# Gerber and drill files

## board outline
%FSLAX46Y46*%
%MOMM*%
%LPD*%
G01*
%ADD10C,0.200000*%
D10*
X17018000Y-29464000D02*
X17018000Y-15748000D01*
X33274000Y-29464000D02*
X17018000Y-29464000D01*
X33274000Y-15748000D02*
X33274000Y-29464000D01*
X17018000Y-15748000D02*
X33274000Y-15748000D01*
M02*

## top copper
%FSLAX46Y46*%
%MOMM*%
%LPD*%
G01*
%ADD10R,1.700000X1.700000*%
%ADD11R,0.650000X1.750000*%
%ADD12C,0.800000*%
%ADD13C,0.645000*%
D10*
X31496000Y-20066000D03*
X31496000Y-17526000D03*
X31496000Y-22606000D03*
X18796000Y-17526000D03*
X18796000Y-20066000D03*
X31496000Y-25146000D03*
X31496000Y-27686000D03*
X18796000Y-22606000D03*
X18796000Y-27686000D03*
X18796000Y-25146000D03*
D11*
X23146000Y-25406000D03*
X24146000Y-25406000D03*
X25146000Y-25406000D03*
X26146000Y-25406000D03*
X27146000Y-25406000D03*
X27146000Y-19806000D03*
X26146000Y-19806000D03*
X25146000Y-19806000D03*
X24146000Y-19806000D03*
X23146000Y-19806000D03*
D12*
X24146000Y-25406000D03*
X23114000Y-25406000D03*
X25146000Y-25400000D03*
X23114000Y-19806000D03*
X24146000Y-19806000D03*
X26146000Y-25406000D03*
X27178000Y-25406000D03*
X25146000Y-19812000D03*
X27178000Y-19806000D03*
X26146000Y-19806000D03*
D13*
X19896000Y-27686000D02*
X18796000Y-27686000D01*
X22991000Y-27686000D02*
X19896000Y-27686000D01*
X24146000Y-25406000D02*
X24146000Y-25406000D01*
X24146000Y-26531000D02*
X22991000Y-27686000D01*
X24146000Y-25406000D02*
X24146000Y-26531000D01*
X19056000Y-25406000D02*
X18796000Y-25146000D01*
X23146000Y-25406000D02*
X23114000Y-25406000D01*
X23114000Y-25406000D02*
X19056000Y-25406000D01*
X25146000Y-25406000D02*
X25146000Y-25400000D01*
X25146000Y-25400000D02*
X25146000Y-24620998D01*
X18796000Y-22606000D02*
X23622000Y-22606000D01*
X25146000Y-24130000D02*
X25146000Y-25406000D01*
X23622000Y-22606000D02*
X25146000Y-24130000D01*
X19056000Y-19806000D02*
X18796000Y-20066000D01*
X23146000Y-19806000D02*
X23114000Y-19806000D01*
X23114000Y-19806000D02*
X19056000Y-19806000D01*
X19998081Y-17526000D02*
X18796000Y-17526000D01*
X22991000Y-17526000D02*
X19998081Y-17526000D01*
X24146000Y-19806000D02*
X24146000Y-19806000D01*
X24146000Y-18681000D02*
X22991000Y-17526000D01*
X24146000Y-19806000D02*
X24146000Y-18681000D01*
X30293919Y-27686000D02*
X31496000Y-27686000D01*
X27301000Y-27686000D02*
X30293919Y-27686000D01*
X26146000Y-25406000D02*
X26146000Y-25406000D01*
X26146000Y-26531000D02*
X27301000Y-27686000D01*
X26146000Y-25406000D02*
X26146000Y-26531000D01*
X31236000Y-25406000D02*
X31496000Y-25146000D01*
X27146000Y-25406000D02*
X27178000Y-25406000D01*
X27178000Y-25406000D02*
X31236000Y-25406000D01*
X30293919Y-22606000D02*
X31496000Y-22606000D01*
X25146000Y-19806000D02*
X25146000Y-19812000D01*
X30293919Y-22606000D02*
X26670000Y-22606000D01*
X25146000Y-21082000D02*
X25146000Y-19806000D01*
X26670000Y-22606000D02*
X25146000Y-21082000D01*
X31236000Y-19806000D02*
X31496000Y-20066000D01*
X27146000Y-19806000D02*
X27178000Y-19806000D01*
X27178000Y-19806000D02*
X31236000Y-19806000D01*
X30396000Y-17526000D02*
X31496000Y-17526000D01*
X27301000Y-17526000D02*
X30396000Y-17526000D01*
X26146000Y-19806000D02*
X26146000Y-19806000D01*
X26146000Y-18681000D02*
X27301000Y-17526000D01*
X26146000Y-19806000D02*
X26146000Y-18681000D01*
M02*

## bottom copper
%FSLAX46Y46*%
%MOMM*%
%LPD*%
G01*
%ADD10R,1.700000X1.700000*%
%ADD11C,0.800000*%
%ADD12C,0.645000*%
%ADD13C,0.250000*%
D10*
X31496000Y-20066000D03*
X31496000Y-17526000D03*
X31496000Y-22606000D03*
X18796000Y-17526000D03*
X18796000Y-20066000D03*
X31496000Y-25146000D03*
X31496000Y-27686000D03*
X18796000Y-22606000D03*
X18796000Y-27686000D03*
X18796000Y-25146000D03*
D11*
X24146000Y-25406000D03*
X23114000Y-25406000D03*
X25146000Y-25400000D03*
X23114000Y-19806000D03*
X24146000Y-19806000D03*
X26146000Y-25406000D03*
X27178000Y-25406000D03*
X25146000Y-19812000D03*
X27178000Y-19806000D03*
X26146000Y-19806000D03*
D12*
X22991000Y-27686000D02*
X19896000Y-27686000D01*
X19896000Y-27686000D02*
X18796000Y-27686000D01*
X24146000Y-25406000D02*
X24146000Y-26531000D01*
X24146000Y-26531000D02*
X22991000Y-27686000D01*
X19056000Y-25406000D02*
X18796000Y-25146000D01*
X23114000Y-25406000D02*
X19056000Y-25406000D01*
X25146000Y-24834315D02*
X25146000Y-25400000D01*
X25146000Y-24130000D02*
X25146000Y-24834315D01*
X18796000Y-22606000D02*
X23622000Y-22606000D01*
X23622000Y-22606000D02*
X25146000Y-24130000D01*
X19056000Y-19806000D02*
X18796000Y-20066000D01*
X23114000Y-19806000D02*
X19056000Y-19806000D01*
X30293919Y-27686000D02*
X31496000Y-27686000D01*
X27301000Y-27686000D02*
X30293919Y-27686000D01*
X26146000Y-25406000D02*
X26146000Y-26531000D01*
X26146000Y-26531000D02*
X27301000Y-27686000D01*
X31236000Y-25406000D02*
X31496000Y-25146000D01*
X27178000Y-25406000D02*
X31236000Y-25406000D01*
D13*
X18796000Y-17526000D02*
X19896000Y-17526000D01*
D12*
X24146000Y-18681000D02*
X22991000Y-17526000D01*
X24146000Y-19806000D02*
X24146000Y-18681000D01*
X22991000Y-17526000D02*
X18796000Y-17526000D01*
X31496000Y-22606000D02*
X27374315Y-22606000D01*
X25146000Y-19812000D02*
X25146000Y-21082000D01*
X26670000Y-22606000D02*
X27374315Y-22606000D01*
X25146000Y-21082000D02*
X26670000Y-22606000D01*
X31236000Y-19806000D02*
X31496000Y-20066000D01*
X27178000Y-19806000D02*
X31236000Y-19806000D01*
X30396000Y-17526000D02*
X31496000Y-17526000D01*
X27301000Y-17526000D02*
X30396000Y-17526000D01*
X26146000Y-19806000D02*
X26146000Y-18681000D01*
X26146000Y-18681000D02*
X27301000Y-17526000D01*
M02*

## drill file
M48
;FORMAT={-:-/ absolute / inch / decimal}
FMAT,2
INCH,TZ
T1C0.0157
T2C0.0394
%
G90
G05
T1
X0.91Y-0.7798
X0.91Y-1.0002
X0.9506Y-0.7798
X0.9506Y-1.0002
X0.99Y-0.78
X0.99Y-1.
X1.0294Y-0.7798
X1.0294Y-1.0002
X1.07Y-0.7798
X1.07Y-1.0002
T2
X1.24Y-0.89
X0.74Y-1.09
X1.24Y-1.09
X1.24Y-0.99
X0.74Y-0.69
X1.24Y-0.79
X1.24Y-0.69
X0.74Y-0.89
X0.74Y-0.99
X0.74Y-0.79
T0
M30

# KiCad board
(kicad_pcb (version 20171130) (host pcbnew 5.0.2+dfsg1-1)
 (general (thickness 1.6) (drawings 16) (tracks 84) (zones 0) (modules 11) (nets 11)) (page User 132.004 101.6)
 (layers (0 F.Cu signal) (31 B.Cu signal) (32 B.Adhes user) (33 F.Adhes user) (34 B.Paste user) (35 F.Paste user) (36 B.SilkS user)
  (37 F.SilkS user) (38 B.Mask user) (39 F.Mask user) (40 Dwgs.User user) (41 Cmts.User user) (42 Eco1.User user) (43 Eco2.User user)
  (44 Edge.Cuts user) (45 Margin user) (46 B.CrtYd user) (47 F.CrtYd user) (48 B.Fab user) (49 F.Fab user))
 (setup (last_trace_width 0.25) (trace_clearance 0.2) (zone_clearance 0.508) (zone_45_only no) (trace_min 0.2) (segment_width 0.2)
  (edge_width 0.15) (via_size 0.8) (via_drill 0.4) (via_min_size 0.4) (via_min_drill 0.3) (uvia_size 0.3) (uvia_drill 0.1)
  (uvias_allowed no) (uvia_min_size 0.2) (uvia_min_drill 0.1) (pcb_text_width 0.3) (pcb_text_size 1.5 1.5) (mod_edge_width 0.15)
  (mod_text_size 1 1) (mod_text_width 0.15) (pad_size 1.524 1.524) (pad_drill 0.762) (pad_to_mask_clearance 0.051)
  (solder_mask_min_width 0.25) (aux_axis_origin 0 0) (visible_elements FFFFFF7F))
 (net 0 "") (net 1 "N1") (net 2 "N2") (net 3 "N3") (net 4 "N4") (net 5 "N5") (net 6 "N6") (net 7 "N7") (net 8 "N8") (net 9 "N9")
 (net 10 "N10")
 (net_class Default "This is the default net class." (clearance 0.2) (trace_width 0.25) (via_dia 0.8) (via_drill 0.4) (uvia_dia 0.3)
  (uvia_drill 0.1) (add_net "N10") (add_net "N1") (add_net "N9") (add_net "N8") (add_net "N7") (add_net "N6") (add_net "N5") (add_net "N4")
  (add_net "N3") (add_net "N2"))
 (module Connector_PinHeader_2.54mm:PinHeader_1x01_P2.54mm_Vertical (layer F.Cu) (at 31.496 20.066)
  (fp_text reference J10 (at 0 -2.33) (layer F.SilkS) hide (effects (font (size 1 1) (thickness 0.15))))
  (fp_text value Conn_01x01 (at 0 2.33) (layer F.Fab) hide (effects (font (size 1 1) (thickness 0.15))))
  (pad 1 thru_hole rect (at 0 0) (size 1.7 1.7) (drill 1) (layers *.Cu *.Mask) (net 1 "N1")))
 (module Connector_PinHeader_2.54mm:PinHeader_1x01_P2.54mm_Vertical (layer F.Cu) (at 31.496 17.526)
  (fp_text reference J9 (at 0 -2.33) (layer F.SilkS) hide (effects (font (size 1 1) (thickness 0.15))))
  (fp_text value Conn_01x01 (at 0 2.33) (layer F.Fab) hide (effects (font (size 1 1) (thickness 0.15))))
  (pad 1 thru_hole rect (at 0 0) (size 1.7 1.7) (drill 1) (layers *.Cu *.Mask) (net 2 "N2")))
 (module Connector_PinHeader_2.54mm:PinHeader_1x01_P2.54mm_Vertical (layer F.Cu) (at 31.496 22.606)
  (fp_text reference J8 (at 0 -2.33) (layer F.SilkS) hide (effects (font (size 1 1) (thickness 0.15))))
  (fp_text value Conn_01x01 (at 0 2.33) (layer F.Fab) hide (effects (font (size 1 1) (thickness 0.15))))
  (pad 1 thru_hole rect (at 0 0) (size 1.7 1.7) (drill 1) (layers *.Cu *.Mask) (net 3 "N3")))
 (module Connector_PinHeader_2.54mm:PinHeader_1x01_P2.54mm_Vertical (layer F.Cu) (at 18.796 17.526)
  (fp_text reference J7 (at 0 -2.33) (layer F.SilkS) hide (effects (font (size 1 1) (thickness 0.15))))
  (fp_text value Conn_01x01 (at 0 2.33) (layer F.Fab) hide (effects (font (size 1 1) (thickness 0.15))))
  (pad 1 thru_hole rect (at 0 0) (size 1.7 1.7) (drill 1) (layers *.Cu *.Mask) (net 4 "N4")))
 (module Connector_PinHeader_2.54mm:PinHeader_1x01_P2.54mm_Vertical (layer F.Cu) (at 18.796 20.066)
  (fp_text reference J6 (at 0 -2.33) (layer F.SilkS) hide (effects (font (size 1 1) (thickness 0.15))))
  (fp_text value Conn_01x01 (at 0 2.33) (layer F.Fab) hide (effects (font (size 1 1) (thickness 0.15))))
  (pad 1 thru_hole rect (at 0 0) (size 1.7 1.7) (drill 1) (layers *.Cu *.Mask) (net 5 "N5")))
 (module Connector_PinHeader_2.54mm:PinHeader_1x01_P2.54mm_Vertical (layer F.Cu) (at 31.496 25.146)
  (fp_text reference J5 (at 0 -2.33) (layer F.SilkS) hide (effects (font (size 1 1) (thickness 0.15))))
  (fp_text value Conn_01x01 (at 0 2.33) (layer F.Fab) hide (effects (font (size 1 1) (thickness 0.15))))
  (pad 1 thru_hole rect (at 0 0) (size 1.7 1.7) (drill 1) (layers *.Cu *.Mask) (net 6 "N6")))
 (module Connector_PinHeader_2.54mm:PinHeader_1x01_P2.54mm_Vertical (layer F.Cu) (at 31.496 27.686)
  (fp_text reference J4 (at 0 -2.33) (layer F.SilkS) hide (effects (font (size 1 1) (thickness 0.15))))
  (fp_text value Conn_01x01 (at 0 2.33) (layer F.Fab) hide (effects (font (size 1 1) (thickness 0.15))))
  (pad 1 thru_hole rect (at 0 0) (size 1.7 1.7) (drill 1) (layers *.Cu *.Mask) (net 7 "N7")))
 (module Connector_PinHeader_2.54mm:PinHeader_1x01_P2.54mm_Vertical (layer F.Cu) (at 18.796 22.606)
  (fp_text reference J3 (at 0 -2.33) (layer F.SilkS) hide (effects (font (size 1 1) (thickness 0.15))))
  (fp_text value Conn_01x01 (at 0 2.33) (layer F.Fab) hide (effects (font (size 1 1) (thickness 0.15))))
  (pad 1 thru_hole rect (at 0 0) (size 1.7 1.7) (drill 1) (layers *.Cu *.Mask) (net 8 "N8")))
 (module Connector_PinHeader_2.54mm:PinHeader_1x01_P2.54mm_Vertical (layer F.Cu) (at 18.796 27.686)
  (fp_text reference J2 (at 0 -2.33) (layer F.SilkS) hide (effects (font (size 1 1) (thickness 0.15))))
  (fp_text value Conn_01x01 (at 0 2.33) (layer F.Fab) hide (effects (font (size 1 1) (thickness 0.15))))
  (pad 1 thru_hole rect (at 0 0) (size 1.7 1.7) (drill 1) (layers *.Cu *.Mask) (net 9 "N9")))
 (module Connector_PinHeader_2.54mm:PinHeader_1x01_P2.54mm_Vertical (layer F.Cu) (at 18.796 25.146)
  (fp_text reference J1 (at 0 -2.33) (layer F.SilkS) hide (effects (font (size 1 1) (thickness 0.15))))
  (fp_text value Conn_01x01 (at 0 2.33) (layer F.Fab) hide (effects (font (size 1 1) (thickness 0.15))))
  (pad 1 thru_hole rect (at 0 0) (size 1.7 1.7) (drill 1) (layers *.Cu *.Mask) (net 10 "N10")))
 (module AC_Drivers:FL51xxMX (layer F.Cu) (at 25.146 22.606)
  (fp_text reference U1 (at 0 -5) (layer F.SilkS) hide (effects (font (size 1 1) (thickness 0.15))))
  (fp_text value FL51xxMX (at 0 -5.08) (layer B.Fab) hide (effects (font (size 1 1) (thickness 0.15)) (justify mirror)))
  (pad 1 smd rect (at -2 2.8) (size 0.65 1.75) (layers F.Cu F.Paste F.Mask) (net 10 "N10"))
  (pad 2 smd rect (at -1 2.8) (size 0.65 1.75) (layers F.Cu F.Paste F.Mask) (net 9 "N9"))
  (pad 3 smd rect (at 0 2.8) (size 0.65 1.75) (layers F.Cu F.Paste F.Mask) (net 8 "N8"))
  (pad 4 smd rect (at 1 2.8) (size 0.65 1.75) (layers F.Cu F.Paste F.Mask) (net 7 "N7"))
  (pad 5 smd rect (at 2 2.8) (size 0.65 1.75) (layers F.Cu F.Paste F.Mask) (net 6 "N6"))
  (pad 6 smd rect (at 2 -2.8) (size 0.65 1.75) (layers F.Cu F.Paste F.Mask) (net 1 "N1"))
  (pad 7 smd rect (at 1 -2.8) (size 0.65 1.75) (layers F.Cu F.Paste F.Mask) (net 2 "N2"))
  (pad 8 smd rect (at 0 -2.8) (size 0.65 1.75) (layers F.Cu F.Paste F.Mask) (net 3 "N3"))
  (pad 9 smd rect (at -1 -2.8) (size 0.65 1.75) (layers F.Cu F.Paste F.Mask) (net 4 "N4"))
  (pad 10 smd rect (at -2 -2.8) (size 0.65 1.75) (layers F.Cu F.Paste F.Mask) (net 5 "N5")))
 (gr_line (start 17.018 29.464) (end 17.018 15.748) (layer Edge.Cuts) (width 0.2))
 (gr_line (start 33.274 29.464) (end 17.018 29.464) (layer Edge.Cuts) (width 0.2))
 (gr_line (start 33.274 15.748) (end 33.274 29.464) (layer Edge.Cuts) (width 0.2))
 (gr_line (start 17.018 15.748) (end 33.274 15.748) (layer Edge.Cuts) (width 0.2))
 (segment (start 19.896 27.686) (end 18.796 27.686) (width 0.645) (layer F.Cu) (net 9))
 (segment (start 22.991 27.686) (end 19.896 27.686) (width 0.645) (layer F.Cu) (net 9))
 (segment (start 24.146 25.406) (end 24.146 25.406) (width 0.645) (layer F.Cu) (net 9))
 (segment (start 24.146 26.531) (end 22.991 27.686) (width 0.645) (layer F.Cu) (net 9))
 (segment (start 24.146 25.406) (end 24.146 26.531) (width 0.645) (layer F.Cu) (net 9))
 (via (at 24.146 25.406) (size 0.8) (drill 0.4) (layers F.Cu B.Cu) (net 9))
 (segment (start 22.991 27.686) (end 19.896 27.686) (width 0.645) (layer B.Cu) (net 9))
 (segment (start 19.896 27.686) (end 18.796 27.686) (width 0.645) (layer B.Cu) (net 9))
 (segment (start 24.146 25.406) (end 24.146 26.531) (width 0.645) (layer B.Cu) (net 9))
 (segment (start 24.146 26.531) (end 22.991 27.686) (width 0.645) (layer B.Cu) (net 9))
 (segment (start 19.056 25.406) (end 18.796 25.146) (width 0.645) (layer F.Cu) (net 10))
 (segment (start 23.146 25.406) (end 23.114 25.406) (width 0.645) (layer F.Cu) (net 10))
 (segment (start 23.114 25.406) (end 19.056 25.406) (width 0.645) (layer F.Cu) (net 10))
 (via (at 23.114 25.406) (size 0.8) (drill 0.4) (layers F.Cu B.Cu) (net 10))
 (segment (start 19.056 25.406) (end 18.796 25.146) (width 0.645) (layer B.Cu) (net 10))
 (segment (start 23.114 25.406) (end 19.056 25.406) (width 0.645) (layer B.Cu) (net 10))
 (segment (start 25.146 25.406) (end 25.146 25.4) (width 0.645) (layer F.Cu) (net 8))
 (segment (start 25.146 25.4) (end 25.146 24.620998) (width 0.645) (layer F.Cu) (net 8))
 (via (at 25.146 25.4) (size 0.8) (drill 0.4) (layers F.Cu B.Cu) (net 8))
 (segment (start 25.146 24.834315) (end 25.146 25.4) (width 0.645) (layer B.Cu) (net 8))
 (segment (start 25.146 24.13) (end 25.146 24.834315) (width 0.645) (layer B.Cu) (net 8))
 (segment (start 18.796 22.606) (end 23.622 22.606) (width 0.645) (layer B.Cu) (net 8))
 (segment (start 23.622 22.606) (end 25.146 24.13) (width 0.645) (layer B.Cu) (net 8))
 (segment (start 18.796 22.606) (end 23.622 22.606) (width 0.645) (layer F.Cu) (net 8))
 (segment (start 25.146 24.13) (end 25.146 25.406) (width 0.645) (layer F.Cu) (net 8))
 (segment (start 23.622 22.606) (end 25.146 24.13) (width 0.645) (layer F.Cu) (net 8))
 (segment (start 19.056 19.806) (end 18.796 20.066) (width 0.645) (layer F.Cu) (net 5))
 (segment (start 23.146 19.806) (end 23.114 19.806) (width 0.645) (layer F.Cu) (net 5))
 (segment (start 23.114 19.806) (end 19.056 19.806) (width 0.645) (layer F.Cu) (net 5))
 (via (at 23.114 19.806) (size 0.8) (drill 0.4) (layers F.Cu B.Cu) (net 5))
 (segment (start 19.056 19.806) (end 18.796 20.066) (width 0.645) (layer B.Cu) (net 5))
 (segment (start 23.114 19.806) (end 19.056 19.806) (width 0.645) (layer B.Cu) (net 5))
 (segment (start 19.998081 17.526) (end 18.796 17.526) (width 0.645) (layer F.Cu) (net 4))
 (segment (start 22.991 17.526) (end 19.998081 17.526) (width 0.645) (layer F.Cu) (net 4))
 (segment (start 24.146 19.806) (end 24.146 19.806) (width 0.645) (layer F.Cu) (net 4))
 (segment (start 24.146 18.681) (end 22.991 17.526) (width 0.645) (layer F.Cu) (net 4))
 (segment (start 24.146 19.806) (end 24.146 18.681) (width 0.645) (layer F.Cu) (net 4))
 (via (at 24.146 19.806) (size 0.8) (drill 0.4) (layers F.Cu B.Cu) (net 4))
 (segment (start 30.293919 27.686) (end 31.496 27.686) (width 0.645) (layer F.Cu) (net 7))
 (segment (start 27.301 27.686) (end 30.293919 27.686) (width 0.645) (layer F.Cu) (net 7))
 (segment (start 26.146 25.406) (end 26.146 25.406) (width 0.645) (layer F.Cu) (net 7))
 (segment (start 26.146 26.531) (end 27.301 27.686) (width 0.645) (layer F.Cu) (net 7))
 (segment (start 26.146 25.406) (end 26.146 26.531) (width 0.645) (layer F.Cu) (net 7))
 (via (at 26.146 25.406) (size 0.8) (drill 0.4) (layers F.Cu B.Cu) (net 7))
 (segment (start 30.293919 27.686) (end 31.496 27.686) (width 0.645) (layer B.Cu) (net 7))
 (segment (start 27.301 27.686) (end 30.293919 27.686) (width 0.645) (layer B.Cu) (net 7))
 (segment (start 26.146 25.406) (end 26.146 26.531) (width 0.645) (layer B.Cu) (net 7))
 (segment (start 26.146 26.531) (end 27.301 27.686) (width 0.645) (layer B.Cu) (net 7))
 (segment (start 31.236 25.406) (end 31.496 25.146) (width 0.645) (layer F.Cu) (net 6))
 (segment (start 27.146 25.406) (end 27.178 25.406) (width 0.645) (layer F.Cu) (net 6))
 (segment (start 27.178 25.406) (end 31.236 25.406) (width 0.645) (layer F.Cu) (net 6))
 (via (at 27.178 25.406) (size 0.8) (drill 0.4) (layers F.Cu B.Cu) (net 6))
 (segment (start 31.236 25.406) (end 31.496 25.146) (width 0.645) (layer B.Cu) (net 6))
 (segment (start 27.178 25.406) (end 31.236 25.406) (width 0.645) (layer B.Cu) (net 6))
 (segment (start 18.796 17.526) (end 19.896 17.526) (width 0.25) (layer B.Cu) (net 4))
 (segment (start 24.146 18.681) (end 22.991 17.526) (width 0.645) (layer B.Cu) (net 4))
 (segment (start 24.146 19.806) (end 24.146 18.681) (width 0.645) (layer B.Cu) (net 4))
 (segment (start 22.991 17.526) (end 18.796 17.526) (width 0.645) (layer B.Cu) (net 4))
 (segment (start 30.293919 22.606) (end 31.496 22.606) (width 0.645) (layer F.Cu) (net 3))
 (segment (start 25.146 19.806) (end 25.146 19.812) (width 0.645) (layer F.Cu) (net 3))
 (via (at 25.146 19.812) (size 0.8) (drill 0.4) (layers F.Cu B.Cu) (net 3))
 (segment (start 31.496 22.606) (end 27.374315 22.606) (width 0.645) (layer B.Cu) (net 3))
 (segment (start 25.146 19.812) (end 25.146 21.082) (width 0.645) (layer B.Cu) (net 3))
 (segment (start 26.67 22.606) (end 27.374315 22.606) (width 0.645) (layer B.Cu) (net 3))
 (segment (start 25.146 21.082) (end 26.67 22.606) (width 0.645) (layer B.Cu) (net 3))
 (segment (start 30.293919 22.606) (end 26.67 22.606) (width 0.645) (layer F.Cu) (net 3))
 (segment (start 25.146 21.082) (end 25.146 19.806) (width 0.645) (layer F.Cu) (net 3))
 (segment (start 26.67 22.606) (end 25.146 21.082) (width 0.645) (layer F.Cu) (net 3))
 (segment (start 31.236 19.806) (end 31.496 20.066) (width 0.645) (layer F.Cu) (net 1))
 (segment (start 27.146 19.806) (end 27.178 19.806) (width 0.645) (layer F.Cu) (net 1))
 (segment (start 27.178 19.806) (end 31.236 19.806) (width 0.645) (layer F.Cu) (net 1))
 (via (at 27.178 19.806) (size 0.8) (drill 0.4) (layers F.Cu B.Cu) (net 1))
 (segment (start 31.236 19.806) (end 31.496 20.066) (width 0.645) (layer B.Cu) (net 1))
 (segment (start 27.178 19.806) (end 31.236 19.806) (width 0.645) (layer B.Cu) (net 1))
 (segment (start 30.396 17.526) (end 31.496 17.526) (width 0.645) (layer F.Cu) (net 2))
 (segment (start 27.301 17.526) (end 30.396 17.526) (width 0.645) (layer F.Cu) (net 2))
 (segment (start 26.146 19.806) (end 26.146 19.806) (width 0.645) (layer F.Cu) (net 2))
 (segment (start 26.146 18.681) (end 27.301 17.526) (width 0.645) (layer F.Cu) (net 2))
 (segment (start 26.146 19.806) (end 26.146 18.681) (width 0.645) (layer F.Cu) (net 2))
 (via (at 26.146 19.806) (size 0.8) (drill 0.4) (layers F.Cu B.Cu) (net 2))
 (segment (start 30.396 17.526) (end 31.496 17.526) (width 0.645) (layer B.Cu) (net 2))
 (segment (start 27.301 17.526) (end 30.396 17.526) (width 0.645) (layer B.Cu) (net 2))
 (segment (start 26.146 19.806) (end 26.146 18.681) (width 0.645) (layer B.Cu) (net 2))
 (segment (start 26.146 18.681) (end 27.301 17.526) (width 0.645) (layer B.Cu) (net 2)))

